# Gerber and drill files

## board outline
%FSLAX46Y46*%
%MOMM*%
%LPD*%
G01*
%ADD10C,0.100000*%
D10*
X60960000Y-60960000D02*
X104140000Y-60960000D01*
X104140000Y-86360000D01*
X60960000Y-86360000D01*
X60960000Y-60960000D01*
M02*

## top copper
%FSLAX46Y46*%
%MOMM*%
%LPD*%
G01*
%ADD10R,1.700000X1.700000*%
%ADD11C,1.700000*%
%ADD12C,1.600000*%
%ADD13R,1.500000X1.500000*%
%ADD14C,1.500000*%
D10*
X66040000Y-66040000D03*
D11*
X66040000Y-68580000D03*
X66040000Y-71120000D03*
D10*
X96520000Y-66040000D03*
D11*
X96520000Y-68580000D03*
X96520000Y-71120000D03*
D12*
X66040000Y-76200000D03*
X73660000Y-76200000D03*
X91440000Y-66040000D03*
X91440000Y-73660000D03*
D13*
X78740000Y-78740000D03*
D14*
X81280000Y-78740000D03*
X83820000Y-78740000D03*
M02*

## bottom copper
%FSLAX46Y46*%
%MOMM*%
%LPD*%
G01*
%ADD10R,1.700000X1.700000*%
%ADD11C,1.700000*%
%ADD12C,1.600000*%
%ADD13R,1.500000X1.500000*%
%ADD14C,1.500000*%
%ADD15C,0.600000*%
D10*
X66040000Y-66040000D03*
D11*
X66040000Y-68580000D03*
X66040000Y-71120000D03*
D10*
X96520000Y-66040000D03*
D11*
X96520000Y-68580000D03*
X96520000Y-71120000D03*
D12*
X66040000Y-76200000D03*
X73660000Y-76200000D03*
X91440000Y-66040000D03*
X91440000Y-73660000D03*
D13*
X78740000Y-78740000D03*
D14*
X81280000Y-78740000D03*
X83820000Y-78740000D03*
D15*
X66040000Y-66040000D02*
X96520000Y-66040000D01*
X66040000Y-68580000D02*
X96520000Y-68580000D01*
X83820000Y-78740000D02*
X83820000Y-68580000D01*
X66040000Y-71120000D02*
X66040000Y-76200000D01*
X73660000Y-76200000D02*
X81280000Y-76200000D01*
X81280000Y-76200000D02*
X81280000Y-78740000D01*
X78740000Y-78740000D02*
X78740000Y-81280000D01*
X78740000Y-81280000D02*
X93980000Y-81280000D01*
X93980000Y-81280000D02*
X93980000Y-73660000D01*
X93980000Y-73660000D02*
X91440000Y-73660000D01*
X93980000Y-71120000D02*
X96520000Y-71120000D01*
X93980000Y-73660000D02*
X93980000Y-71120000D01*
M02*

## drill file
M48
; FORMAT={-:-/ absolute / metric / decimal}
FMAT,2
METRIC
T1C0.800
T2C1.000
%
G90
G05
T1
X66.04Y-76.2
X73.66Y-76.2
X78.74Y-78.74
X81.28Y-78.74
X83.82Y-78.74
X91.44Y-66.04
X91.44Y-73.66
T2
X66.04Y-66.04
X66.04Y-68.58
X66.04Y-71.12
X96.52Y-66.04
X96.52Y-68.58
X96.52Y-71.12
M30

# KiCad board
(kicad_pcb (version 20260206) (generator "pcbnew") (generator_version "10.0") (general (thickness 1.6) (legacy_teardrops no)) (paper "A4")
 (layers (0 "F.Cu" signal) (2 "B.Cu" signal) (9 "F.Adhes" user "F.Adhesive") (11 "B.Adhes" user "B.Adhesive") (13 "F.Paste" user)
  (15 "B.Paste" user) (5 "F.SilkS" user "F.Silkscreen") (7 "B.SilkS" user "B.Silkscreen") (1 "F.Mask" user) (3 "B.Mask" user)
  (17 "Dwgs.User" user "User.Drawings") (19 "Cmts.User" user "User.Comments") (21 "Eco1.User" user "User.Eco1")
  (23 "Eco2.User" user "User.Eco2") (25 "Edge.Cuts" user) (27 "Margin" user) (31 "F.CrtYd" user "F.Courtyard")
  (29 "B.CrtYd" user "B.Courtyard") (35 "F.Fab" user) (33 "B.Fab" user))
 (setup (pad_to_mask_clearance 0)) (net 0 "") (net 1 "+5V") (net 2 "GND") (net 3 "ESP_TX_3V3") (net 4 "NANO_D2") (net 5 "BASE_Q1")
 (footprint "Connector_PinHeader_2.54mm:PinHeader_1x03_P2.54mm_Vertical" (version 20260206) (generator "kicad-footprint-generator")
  (layer "F.Cu") (at 66.040 66.040 0)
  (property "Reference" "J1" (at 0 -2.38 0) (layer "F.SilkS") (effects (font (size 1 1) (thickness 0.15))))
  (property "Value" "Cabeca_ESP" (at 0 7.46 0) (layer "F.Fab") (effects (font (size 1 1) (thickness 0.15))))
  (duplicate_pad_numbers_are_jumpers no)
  (pad "1" thru_hole rect (at 0 0) (size 1.7 1.7) (drill 1) (layers "*.Cu" "*.Mask") (remove_unused_layers no) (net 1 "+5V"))
  (pad "2" thru_hole circle (at 0 2.54) (size 1.7 1.7) (drill 1) (layers "*.Cu" "*.Mask") (remove_unused_layers no) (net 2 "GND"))
  (pad "3" thru_hole circle (at 0 5.08) (size 1.7 1.7) (drill 1) (layers "*.Cu" "*.Mask") (remove_unused_layers no) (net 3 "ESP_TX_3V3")))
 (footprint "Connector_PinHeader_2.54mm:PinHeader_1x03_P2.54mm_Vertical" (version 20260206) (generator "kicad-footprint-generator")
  (layer "F.Cu") (at 96.520 66.040 0)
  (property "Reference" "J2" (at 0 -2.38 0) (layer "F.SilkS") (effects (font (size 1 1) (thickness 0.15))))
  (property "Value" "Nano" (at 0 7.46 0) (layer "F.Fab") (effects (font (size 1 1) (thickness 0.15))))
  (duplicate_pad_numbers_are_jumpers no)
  (pad "1" thru_hole rect (at 0 0) (size 1.7 1.7) (drill 1) (layers "*.Cu" "*.Mask") (remove_unused_layers no) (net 1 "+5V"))
  (pad "2" thru_hole circle (at 0 2.54) (size 1.7 1.7) (drill 1) (layers "*.Cu" "*.Mask") (remove_unused_layers no) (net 2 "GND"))
  (pad "3" thru_hole circle (at 0 5.08) (size 1.7 1.7) (drill 1) (layers "*.Cu" "*.Mask") (remove_unused_layers no) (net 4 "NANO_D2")))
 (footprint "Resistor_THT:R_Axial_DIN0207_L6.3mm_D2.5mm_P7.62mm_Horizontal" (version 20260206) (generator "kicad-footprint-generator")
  (layer "F.Cu") (at 66.040 76.200 0)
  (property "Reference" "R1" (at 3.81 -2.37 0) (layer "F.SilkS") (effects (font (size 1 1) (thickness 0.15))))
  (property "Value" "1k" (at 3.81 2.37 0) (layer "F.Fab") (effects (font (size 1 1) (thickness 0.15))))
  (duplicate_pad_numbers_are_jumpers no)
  (pad "1" thru_hole circle (at 0 0) (size 1.6 1.6) (drill 0.8) (layers "*.Cu" "*.Mask") (remove_unused_layers no) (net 3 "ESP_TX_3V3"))
  (pad "2" thru_hole circle (at 7.62 0) (size 1.6 1.6) (drill 0.8) (layers "*.Cu" "*.Mask") (remove_unused_layers no) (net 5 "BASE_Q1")))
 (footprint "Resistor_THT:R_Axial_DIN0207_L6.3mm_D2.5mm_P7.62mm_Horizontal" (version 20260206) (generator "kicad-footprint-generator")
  (layer "F.Cu") (at 91.440 66.040 270)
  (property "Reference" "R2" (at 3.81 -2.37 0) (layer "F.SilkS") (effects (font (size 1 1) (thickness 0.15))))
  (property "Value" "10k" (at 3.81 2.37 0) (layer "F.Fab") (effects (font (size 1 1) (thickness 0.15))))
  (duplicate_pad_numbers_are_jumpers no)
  (pad "1" thru_hole circle (at 0 0) (size 1.6 1.6) (drill 0.8) (layers "*.Cu" "*.Mask") (remove_unused_layers no) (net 1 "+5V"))
  (pad "2" thru_hole circle (at 7.62 0) (size 1.6 1.6) (drill 0.8) (layers "*.Cu" "*.Mask") (remove_unused_layers no) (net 4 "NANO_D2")))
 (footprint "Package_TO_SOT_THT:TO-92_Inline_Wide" (layer "F.Cu") (at 78.740 78.740 0)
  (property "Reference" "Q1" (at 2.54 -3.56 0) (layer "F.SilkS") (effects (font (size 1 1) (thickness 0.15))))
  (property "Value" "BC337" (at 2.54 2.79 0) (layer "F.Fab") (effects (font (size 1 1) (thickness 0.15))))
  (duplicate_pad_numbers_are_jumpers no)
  (pad "1" thru_hole rect (at 0 0) (size 1.5 1.5) (drill 0.8) (layers "*.Cu" "*.Mask") (remove_unused_layers no) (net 4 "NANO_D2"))
  (pad "2" thru_hole circle (at 2.54 0) (size 1.5 1.5) (drill 0.8) (layers "*.Cu" "*.Mask") (remove_unused_layers no) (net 5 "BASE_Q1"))
  (pad "3" thru_hole circle (at 5.08 0) (size 1.5 1.5) (drill 0.8) (layers "*.Cu" "*.Mask") (remove_unused_layers no) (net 2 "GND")))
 (segment (start 66.040 66.040) (end 96.520 66.040) (width 0.6) (layer "B.Cu") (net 1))
 (segment (start 66.040 68.580) (end 96.520 68.580) (width 0.6) (layer "B.Cu") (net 2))
 (segment (start 83.820 78.740) (end 83.820 68.580) (width 0.6) (layer "B.Cu") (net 2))
 (segment (start 66.040 71.120) (end 66.040 76.200) (width 0.6) (layer "B.Cu") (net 3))
 (segment (start 73.660 76.200) (end 81.280 76.200) (width 0.6) (layer "B.Cu") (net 5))
 (segment (start 81.280 76.200) (end 81.280 78.740) (width 0.6) (layer "B.Cu") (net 5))
 (segment (start 78.740 78.740) (end 78.740 81.280) (width 0.6) (layer "B.Cu") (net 4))
 (segment (start 78.740 81.280) (end 93.980 81.280) (width 0.6) (layer "B.Cu") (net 4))
 (segment (start 93.980 81.280) (end 93.980 73.660) (width 0.6) (layer "B.Cu") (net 4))
 (segment (start 93.980 73.660) (end 91.440 73.660) (width 0.6) (layer "B.Cu") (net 4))
 (segment (start 93.980 71.120) (end 96.520 71.120) (width 0.6) (layer "B.Cu") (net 4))
 (segment (start 93.980 73.660) (end 93.980 71.120) (width 0.6) (layer "B.Cu") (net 4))
 (gr_rect (start 60.960 60.960) (end 104.140 86.360) (stroke (width 0.1) (type default)) (fill no) (layer "Edge.Cuts")))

